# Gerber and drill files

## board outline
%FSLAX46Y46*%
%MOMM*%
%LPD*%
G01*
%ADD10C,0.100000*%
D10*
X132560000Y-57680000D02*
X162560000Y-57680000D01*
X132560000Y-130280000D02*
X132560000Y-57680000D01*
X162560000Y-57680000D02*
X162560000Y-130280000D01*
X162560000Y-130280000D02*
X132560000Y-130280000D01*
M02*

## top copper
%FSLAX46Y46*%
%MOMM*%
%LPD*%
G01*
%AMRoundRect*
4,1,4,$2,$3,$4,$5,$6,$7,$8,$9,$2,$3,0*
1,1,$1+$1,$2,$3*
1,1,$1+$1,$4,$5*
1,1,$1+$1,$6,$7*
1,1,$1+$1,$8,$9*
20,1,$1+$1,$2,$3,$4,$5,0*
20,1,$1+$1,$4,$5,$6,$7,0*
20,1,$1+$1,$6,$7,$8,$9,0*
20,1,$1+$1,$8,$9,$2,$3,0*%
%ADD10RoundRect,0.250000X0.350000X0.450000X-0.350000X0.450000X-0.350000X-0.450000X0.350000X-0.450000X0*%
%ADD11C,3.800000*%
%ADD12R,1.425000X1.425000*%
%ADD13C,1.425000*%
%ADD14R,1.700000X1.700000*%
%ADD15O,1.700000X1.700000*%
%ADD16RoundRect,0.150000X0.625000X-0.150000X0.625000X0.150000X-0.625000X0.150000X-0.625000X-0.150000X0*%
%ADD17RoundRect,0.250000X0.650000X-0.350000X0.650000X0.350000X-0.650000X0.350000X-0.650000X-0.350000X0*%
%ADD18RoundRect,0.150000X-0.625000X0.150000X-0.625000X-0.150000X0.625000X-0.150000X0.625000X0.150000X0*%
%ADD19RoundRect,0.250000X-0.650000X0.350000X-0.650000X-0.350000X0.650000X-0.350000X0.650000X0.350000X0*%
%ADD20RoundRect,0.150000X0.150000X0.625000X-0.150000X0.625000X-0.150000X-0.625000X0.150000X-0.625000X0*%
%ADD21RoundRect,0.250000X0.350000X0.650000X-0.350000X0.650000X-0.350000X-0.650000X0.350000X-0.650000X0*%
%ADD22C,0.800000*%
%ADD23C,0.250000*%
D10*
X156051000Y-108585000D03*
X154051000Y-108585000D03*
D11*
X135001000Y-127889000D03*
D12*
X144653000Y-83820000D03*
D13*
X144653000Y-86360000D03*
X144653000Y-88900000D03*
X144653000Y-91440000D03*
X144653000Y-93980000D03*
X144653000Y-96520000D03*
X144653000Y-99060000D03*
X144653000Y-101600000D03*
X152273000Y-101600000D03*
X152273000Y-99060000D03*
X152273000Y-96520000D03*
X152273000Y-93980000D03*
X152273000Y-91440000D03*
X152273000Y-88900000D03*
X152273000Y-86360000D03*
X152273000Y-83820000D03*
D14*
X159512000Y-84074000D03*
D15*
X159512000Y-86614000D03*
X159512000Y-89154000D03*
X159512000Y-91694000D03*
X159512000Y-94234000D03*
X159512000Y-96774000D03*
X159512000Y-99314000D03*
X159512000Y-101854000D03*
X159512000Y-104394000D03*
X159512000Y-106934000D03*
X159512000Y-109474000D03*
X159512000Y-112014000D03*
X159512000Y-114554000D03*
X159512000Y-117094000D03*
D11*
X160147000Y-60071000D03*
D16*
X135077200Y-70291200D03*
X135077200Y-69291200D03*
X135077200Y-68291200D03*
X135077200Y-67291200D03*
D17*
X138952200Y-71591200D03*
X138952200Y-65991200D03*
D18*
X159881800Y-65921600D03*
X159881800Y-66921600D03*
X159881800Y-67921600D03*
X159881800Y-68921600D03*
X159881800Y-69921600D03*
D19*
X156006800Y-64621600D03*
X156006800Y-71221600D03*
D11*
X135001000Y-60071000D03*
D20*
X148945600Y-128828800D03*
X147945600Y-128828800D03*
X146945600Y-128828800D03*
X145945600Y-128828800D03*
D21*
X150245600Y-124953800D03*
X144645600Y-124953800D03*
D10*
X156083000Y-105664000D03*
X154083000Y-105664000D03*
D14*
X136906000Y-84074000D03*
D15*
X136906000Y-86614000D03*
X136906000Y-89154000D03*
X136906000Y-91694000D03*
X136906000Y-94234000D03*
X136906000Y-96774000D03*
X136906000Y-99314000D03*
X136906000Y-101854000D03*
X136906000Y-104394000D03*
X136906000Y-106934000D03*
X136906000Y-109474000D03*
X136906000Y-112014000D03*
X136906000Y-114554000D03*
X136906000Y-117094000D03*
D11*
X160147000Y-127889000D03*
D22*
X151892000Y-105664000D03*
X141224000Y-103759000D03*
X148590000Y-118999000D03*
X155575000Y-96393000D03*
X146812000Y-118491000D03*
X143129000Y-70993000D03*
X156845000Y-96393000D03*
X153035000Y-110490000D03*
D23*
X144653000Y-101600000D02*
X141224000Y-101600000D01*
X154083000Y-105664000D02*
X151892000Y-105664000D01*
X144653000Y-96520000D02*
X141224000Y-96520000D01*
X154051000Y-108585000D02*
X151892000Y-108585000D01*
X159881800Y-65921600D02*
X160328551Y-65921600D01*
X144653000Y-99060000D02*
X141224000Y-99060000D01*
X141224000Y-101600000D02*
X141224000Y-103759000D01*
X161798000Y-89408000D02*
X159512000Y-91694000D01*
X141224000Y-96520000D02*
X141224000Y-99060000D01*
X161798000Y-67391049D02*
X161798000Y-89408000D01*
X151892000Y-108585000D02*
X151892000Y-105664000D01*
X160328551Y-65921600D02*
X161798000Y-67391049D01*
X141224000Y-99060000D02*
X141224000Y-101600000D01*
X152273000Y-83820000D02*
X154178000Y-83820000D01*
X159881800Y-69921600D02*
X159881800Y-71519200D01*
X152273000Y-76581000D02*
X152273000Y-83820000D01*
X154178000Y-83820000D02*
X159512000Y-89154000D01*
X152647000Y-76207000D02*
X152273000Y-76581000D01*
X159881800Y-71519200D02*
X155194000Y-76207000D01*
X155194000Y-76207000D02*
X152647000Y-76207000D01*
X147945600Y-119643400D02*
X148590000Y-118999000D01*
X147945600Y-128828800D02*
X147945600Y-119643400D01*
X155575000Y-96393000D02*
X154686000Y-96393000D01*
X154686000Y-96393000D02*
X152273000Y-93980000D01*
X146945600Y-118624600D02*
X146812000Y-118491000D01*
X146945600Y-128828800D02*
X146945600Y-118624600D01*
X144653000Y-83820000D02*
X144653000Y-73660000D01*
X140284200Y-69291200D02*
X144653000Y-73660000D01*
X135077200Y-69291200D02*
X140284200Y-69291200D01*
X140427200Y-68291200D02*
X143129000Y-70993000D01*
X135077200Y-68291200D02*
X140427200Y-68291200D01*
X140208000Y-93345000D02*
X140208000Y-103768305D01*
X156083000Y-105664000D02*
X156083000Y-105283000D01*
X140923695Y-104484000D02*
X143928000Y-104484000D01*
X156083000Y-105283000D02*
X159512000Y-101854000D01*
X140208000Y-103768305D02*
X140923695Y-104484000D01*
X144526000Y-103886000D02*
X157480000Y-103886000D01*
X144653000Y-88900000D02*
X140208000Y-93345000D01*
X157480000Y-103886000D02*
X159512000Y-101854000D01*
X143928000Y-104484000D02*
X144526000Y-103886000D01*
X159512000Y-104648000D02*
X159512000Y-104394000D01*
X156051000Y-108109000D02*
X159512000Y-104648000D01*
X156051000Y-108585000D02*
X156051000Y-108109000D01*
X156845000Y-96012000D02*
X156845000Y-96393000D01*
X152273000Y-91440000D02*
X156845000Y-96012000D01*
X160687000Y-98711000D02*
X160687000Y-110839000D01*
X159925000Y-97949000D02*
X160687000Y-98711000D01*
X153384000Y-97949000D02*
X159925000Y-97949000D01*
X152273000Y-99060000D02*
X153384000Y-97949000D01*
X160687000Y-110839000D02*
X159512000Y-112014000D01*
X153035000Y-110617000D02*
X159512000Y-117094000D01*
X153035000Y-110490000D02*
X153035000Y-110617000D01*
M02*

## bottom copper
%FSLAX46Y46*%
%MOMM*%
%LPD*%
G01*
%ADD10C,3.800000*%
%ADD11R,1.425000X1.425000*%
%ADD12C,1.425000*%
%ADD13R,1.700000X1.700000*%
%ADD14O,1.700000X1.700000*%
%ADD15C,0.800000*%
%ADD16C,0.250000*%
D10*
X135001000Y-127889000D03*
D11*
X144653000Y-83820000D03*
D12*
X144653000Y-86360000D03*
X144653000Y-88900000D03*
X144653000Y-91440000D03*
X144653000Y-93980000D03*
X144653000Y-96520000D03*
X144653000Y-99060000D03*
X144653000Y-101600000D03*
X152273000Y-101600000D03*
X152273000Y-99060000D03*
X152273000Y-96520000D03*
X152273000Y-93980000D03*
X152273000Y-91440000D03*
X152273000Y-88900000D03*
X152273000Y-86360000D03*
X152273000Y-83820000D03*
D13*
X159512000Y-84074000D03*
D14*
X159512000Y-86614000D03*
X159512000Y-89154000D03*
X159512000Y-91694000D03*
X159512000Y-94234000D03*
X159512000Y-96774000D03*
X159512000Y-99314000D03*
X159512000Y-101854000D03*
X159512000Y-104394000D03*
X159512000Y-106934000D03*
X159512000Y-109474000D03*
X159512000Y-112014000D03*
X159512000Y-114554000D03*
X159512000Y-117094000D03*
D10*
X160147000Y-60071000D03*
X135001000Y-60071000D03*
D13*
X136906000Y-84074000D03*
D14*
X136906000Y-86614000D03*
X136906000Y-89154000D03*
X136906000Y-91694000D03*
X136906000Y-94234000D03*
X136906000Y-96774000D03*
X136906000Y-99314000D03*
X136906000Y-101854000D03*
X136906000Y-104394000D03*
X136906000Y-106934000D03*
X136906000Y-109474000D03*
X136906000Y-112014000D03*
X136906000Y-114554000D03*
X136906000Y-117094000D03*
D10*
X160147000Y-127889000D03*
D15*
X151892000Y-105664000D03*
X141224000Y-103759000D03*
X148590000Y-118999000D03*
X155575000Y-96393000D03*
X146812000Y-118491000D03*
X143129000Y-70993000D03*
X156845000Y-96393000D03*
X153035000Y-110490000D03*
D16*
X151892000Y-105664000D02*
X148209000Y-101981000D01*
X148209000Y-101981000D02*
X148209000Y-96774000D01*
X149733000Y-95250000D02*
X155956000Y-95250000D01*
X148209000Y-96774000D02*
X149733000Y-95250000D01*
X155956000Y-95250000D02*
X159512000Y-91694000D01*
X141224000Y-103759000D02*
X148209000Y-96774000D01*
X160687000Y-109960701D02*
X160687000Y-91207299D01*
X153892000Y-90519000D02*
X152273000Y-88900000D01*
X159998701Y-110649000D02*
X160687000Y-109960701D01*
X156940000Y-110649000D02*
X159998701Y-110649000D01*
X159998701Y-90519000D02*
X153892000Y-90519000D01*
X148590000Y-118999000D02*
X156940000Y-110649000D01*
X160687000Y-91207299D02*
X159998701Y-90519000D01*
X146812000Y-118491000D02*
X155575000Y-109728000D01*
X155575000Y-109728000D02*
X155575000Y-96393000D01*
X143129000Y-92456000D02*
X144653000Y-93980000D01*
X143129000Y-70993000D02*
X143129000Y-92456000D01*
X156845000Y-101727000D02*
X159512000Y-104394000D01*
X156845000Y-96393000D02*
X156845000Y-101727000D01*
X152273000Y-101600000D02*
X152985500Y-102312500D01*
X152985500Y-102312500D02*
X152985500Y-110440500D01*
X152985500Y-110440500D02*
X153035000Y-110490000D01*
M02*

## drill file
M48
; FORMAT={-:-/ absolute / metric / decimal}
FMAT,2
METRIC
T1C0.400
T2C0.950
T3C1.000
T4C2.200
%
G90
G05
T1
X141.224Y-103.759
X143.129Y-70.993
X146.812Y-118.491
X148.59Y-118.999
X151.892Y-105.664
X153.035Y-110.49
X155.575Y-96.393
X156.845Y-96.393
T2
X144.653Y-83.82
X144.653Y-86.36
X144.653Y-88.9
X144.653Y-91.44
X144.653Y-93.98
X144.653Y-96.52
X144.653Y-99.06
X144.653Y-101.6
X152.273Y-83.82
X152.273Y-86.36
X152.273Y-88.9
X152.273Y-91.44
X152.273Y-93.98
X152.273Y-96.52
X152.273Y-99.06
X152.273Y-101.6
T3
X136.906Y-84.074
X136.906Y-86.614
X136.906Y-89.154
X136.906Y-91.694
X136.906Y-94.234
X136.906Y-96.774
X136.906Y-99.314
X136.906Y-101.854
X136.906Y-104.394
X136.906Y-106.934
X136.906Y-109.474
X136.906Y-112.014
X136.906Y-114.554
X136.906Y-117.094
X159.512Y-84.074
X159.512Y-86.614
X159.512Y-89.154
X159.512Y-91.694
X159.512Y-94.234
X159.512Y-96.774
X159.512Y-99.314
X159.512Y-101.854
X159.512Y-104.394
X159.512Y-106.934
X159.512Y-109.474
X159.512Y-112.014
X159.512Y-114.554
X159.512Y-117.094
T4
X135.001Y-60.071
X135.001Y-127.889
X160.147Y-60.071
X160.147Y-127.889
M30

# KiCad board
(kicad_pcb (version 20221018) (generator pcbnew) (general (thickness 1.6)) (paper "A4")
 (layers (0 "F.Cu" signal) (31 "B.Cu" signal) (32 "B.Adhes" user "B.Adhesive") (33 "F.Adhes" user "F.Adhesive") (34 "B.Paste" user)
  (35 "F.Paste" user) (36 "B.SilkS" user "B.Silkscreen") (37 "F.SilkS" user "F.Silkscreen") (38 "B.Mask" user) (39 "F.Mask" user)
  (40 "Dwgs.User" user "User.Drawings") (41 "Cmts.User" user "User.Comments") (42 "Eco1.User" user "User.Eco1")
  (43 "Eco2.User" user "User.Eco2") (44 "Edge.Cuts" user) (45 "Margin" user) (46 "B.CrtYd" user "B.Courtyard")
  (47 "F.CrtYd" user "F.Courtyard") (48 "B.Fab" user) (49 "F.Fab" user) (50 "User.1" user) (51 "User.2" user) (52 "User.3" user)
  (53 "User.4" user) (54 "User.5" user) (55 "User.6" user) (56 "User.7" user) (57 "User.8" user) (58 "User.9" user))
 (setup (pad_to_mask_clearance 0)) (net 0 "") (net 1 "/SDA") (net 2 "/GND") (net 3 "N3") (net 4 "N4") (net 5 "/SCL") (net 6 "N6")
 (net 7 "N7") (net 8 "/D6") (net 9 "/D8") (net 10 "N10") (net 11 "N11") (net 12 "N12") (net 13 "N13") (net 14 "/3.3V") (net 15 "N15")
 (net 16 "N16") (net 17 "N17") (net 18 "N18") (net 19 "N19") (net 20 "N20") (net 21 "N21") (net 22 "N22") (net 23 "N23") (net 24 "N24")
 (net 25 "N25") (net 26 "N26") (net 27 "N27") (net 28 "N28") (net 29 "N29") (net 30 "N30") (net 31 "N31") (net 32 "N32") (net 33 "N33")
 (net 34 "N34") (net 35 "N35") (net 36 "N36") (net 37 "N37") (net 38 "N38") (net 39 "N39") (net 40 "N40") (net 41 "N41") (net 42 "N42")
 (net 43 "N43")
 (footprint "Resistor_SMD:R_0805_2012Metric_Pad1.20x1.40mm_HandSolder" (layer "F.Cu") (at 155.051 108.585 180)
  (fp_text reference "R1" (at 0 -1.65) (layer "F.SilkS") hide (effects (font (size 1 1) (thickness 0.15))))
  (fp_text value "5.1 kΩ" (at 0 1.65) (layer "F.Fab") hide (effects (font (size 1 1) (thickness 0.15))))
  (pad "1" smd roundrect (at -1 0 180) (size 1.2 1.4) (layers "F.Cu" "F.Paste" "F.Mask") (roundrect_rratio 0.2083333333) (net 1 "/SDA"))
  (pad "2" smd roundrect (at 1 0 180) (size 1.2 1.4) (layers "F.Cu" "F.Paste" "F.Mask") (roundrect_rratio 0.2083333333) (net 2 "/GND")))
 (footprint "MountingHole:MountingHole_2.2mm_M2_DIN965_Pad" (layer "F.Cu") (at 135.001 127.889)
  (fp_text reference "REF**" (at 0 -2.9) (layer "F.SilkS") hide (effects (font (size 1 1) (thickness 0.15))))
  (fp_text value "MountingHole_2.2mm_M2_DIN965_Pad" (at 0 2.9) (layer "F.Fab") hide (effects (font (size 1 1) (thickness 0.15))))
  (pad "1" thru_hole circle (at 0 0) (size 3.8 3.8) (drill 2.2) (layers "*.Cu" "*.Mask")))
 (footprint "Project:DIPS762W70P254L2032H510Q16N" (layer "F.Cu") (at 144.653 83.82)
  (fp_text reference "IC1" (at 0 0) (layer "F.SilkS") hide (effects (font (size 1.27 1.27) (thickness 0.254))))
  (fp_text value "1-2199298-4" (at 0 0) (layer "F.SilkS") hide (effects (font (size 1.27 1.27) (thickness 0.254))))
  (pad "1" thru_hole rect (at 0 0) (size 1.425 1.425) (drill 0.95) (layers "*.Cu" "*.Mask") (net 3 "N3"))
  (pad "2" thru_hole circle (at 0 2.54) (size 1.425 1.425) (drill 0.95) (layers "*.Cu" "*.Mask") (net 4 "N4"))
  (pad "3" thru_hole circle (at 0 5.08) (size 1.425 1.425) (drill 0.95) (layers "*.Cu" "*.Mask") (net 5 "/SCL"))
  (pad "4" thru_hole circle (at 0 7.62) (size 1.425 1.425) (drill 0.95) (layers "*.Cu" "*.Mask") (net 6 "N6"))
  (pad "5" thru_hole circle (at 0 10.16) (size 1.425 1.425) (drill 0.95) (layers "*.Cu" "*.Mask") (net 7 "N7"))
  (pad "6" thru_hole circle (at 0 12.7) (size 1.425 1.425) (drill 0.95) (layers "*.Cu" "*.Mask") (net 2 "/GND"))
  (pad "7" thru_hole circle (at 0 15.24) (size 1.425 1.425) (drill 0.95) (layers "*.Cu" "*.Mask") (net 2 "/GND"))
  (pad "8" thru_hole circle (at 0 17.78) (size 1.425 1.425) (drill 0.95) (layers "*.Cu" "*.Mask") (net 2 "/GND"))
  (pad "9" thru_hole circle (at 7.62 17.78) (size 1.425 1.425) (drill 0.95) (layers "*.Cu" "*.Mask") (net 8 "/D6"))
  (pad "10" thru_hole circle (at 7.62 15.24) (size 1.425 1.425) (drill 0.95) (layers "*.Cu" "*.Mask") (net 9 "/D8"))
  (pad "11" thru_hole circle (at 7.62 12.7) (size 1.425 1.425) (drill 0.95) (layers "*.Cu" "*.Mask") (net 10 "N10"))
  (pad "12" thru_hole circle (at 7.62 10.16) (size 1.425 1.425) (drill 0.95) (layers "*.Cu" "*.Mask") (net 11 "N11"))
  (pad "13" thru_hole circle (at 7.62 7.62) (size 1.425 1.425) (drill 0.95) (layers "*.Cu" "*.Mask") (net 1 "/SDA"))
  (pad "14" thru_hole circle (at 7.62 5.08) (size 1.425 1.425) (drill 0.95) (layers "*.Cu" "*.Mask") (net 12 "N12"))
  (pad "15" thru_hole circle (at 7.62 2.54) (size 1.425 1.425) (drill 0.95) (layers "*.Cu" "*.Mask") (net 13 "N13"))
  (pad "16" thru_hole circle (at 7.62 0) (size 1.425 1.425) (drill 0.95) (layers "*.Cu" "*.Mask") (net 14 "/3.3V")))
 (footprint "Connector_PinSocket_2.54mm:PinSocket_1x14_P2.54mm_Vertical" (layer "F.Cu") (at 159.512 84.074)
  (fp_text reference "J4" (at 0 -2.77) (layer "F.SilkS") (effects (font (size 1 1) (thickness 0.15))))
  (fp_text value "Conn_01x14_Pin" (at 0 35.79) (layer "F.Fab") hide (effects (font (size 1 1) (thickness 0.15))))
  (pad "1" thru_hole rect (at 0 0) (size 1.7 1.7) (drill 1) (layers "*.Cu" "*.Mask") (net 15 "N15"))
  (pad "2" thru_hole oval (at 0 2.54) (size 1.7 1.7) (drill 1) (layers "*.Cu" "*.Mask") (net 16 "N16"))
  (pad "3" thru_hole oval (at 0 5.08) (size 1.7 1.7) (drill 1) (layers "*.Cu" "*.Mask") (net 14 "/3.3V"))
  (pad "4" thru_hole oval (at 0 7.62) (size 1.7 1.7) (drill 1) (layers "*.Cu" "*.Mask") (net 2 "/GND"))
  (pad "5" thru_hole oval (at 0 10.16) (size 1.7 1.7) (drill 1) (layers "*.Cu" "*.Mask") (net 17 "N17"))
  (pad "6" thru_hole oval (at 0 12.7) (size 1.7 1.7) (drill 1) (layers "*.Cu" "*.Mask") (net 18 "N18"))
  (pad "7" thru_hole oval (at 0 15.24) (size 1.7 1.7) (drill 1) (layers "*.Cu" "*.Mask") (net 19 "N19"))
  (pad "8" thru_hole oval (at 0 17.78) (size 1.7 1.7) (drill 1) (layers "*.Cu" "*.Mask") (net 5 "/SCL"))
  (pad "9" thru_hole oval (at 0 20.32) (size 1.7 1.7) (drill 1) (layers "*.Cu" "*.Mask") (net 1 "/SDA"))
  (pad "10" thru_hole oval (at 0 22.86) (size 1.7 1.7) (drill 1) (layers "*.Cu" "*.Mask") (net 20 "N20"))
  (pad "11" thru_hole oval (at 0 25.4) (size 1.7 1.7) (drill 1) (layers "*.Cu" "*.Mask") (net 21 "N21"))
  (pad "12" thru_hole oval (at 0 27.94) (size 1.7 1.7) (drill 1) (layers "*.Cu" "*.Mask") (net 9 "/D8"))
  (pad "13" thru_hole oval (at 0 30.48) (size 1.7 1.7) (drill 1) (layers "*.Cu" "*.Mask") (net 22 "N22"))
  (pad "14" thru_hole oval (at 0 33.02) (size 1.7 1.7) (drill 1) (layers "*.Cu" "*.Mask") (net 8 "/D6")))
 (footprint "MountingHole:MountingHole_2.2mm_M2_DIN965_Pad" (layer "F.Cu") (at 160.147 60.071)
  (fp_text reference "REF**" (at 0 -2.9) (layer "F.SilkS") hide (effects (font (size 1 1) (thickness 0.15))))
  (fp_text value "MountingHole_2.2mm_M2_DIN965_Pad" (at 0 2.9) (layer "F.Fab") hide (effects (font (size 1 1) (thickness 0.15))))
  (pad "1" thru_hole circle (at 0 0) (size 3.8 3.8) (drill 2.2) (layers "*.Cu" "*.Mask")))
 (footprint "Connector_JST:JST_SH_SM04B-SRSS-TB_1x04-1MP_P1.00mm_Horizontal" (layer "F.Cu") (at 137.0772 68.7912 90)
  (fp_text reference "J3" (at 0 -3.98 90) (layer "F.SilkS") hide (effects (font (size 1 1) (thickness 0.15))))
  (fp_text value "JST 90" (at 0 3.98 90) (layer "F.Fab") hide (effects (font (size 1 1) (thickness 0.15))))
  (pad "1" smd roundrect (at -1.5 -2 90) (size 0.6 1.55) (layers "F.Cu" "F.Paste" "F.Mask") (roundrect_rratio 0.25) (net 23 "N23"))
  (pad "2" smd roundrect (at -0.5 -2 90) (size 0.6 1.55) (layers "F.Cu" "F.Paste" "F.Mask") (roundrect_rratio 0.25) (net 3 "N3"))
  (pad "3" smd roundrect (at 0.5 -2 90) (size 0.6 1.55) (layers "F.Cu" "F.Paste" "F.Mask") (roundrect_rratio 0.25) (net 7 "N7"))
  (pad "4" smd roundrect (at 1.5 -2 90) (size 0.6 1.55) (layers "F.Cu" "F.Paste" "F.Mask") (roundrect_rratio 0.25) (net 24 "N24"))
  (pad "MP" smd roundrect (at -2.8 1.875 90) (size 1.2 1.8) (layers "F.Cu" "F.Paste" "F.Mask") (roundrect_rratio 0.208333))
  (pad "MP" smd roundrect (at 2.8 1.875 90) (size 1.2 1.8) (layers "F.Cu" "F.Paste" "F.Mask") (roundrect_rratio 0.208333)))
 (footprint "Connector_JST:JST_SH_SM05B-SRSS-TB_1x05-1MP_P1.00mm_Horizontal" (layer "F.Cu") (at 157.8818 67.9216 -90)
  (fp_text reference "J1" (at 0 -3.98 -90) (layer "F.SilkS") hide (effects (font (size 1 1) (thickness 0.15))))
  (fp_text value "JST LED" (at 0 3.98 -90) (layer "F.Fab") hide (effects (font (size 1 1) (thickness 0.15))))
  (pad "1" smd roundrect (at -2 -2 270) (size 0.6 1.55) (layers "F.Cu" "F.Paste" "F.Mask") (roundrect_rratio 0.25) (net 2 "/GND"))
  (pad "2" smd roundrect (at -1 -2 270) (size 0.6 1.55) (layers "F.Cu" "F.Paste" "F.Mask") (roundrect_rratio 0.25) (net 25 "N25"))
  (pad "3" smd roundrect (at 0 -2 270) (size 0.6 1.55) (layers "F.Cu" "F.Paste" "F.Mask") (roundrect_rratio 0.25) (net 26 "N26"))
  (pad "4" smd roundrect (at 1 -2 270) (size 0.6 1.55) (layers "F.Cu" "F.Paste" "F.Mask") (roundrect_rratio 0.25) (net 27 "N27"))
  (pad "5" smd roundrect (at 2 -2 270) (size 0.6 1.55) (layers "F.Cu" "F.Paste" "F.Mask") (roundrect_rratio 0.25) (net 14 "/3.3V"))
  (pad "MP" smd roundrect (at -3.3 1.875 270) (size 1.2 1.8) (layers "F.Cu" "F.Paste" "F.Mask") (roundrect_rratio 0.208333))
  (pad "MP" smd roundrect (at 3.3 1.875 270) (size 1.2 1.8) (layers "F.Cu" "F.Paste" "F.Mask") (roundrect_rratio 0.208333)))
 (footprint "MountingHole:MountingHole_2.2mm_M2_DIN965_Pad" (layer "F.Cu") (at 135.001 60.071)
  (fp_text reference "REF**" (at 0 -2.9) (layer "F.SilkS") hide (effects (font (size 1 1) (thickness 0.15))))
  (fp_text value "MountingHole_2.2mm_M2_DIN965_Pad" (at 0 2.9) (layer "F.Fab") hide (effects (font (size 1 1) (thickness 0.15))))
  (pad "1" thru_hole circle (at 0 0) (size 3.8 3.8) (drill 2.2) (layers "*.Cu" "*.Mask")))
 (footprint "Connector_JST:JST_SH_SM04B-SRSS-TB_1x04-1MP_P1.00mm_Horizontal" (layer "F.Cu") (at 147.4456 126.8288 180)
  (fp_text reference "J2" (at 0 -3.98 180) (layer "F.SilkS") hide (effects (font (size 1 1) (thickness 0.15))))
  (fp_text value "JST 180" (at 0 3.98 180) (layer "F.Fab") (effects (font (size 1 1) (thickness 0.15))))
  (pad "1" smd roundrect (at -1.5 -2 180) (size 0.6 1.55) (layers "F.Cu" "F.Paste" "F.Mask") (roundrect_rratio 0.25) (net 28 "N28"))
  (pad "2" smd roundrect (at -0.5 -2 180) (size 0.6 1.55) (layers "F.Cu" "F.Paste" "F.Mask") (roundrect_rratio 0.25) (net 12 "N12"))
  (pad "3" smd roundrect (at 0.5 -2 180) (size 0.6 1.55) (layers "F.Cu" "F.Paste" "F.Mask") (roundrect_rratio 0.25) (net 11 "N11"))
  (pad "4" smd roundrect (at 1.5 -2 180) (size 0.6 1.55) (layers "F.Cu" "F.Paste" "F.Mask") (roundrect_rratio 0.25) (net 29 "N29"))
  (pad "MP" smd roundrect (at -2.8 1.875 180) (size 1.2 1.8) (layers "F.Cu" "F.Paste" "F.Mask") (roundrect_rratio 0.208333))
  (pad "MP" smd roundrect (at 2.8 1.875 180) (size 1.2 1.8) (layers "F.Cu" "F.Paste" "F.Mask") (roundrect_rratio 0.208333)))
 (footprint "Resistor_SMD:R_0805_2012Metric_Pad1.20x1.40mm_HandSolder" (layer "F.Cu") (at 155.083 105.664 180)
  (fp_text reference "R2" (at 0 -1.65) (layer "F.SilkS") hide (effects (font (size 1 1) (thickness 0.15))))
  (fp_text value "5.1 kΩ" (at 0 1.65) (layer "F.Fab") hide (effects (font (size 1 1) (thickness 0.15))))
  (pad "1" smd roundrect (at -1 0 180) (size 1.2 1.4) (layers "F.Cu" "F.Paste" "F.Mask") (roundrect_rratio 0.2083333333) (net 5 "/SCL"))
  (pad "2" smd roundrect (at 1 0 180) (size 1.2 1.4) (layers "F.Cu" "F.Paste" "F.Mask") (roundrect_rratio 0.2083333333) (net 2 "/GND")))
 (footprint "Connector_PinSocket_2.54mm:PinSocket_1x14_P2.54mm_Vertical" (layer "F.Cu") (at 136.906 84.074)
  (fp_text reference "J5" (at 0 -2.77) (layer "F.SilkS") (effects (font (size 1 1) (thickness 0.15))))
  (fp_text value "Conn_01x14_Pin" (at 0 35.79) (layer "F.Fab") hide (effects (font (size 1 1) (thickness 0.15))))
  (pad "1" thru_hole rect (at 0 0) (size 1.7 1.7) (drill 1) (layers "*.Cu" "*.Mask") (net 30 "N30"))
  (pad "2" thru_hole oval (at 0 2.54) (size 1.7 1.7) (drill 1) (layers "*.Cu" "*.Mask") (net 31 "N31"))
  (pad "3" thru_hole oval (at 0 5.08) (size 1.7 1.7) (drill 1) (layers "*.Cu" "*.Mask") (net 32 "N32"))
  (pad "4" thru_hole oval (at 0 7.62) (size 1.7 1.7) (drill 1) (layers "*.Cu" "*.Mask") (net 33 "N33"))
  (pad "5" thru_hole oval (at 0 10.16) (size 1.7 1.7) (drill 1) (layers "*.Cu" "*.Mask") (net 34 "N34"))
  (pad "6" thru_hole oval (at 0 12.7) (size 1.7 1.7) (drill 1) (layers "*.Cu" "*.Mask") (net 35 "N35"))
  (pad "7" thru_hole oval (at 0 15.24) (size 1.7 1.7) (drill 1) (layers "*.Cu" "*.Mask") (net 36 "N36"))
  (pad "8" thru_hole oval (at 0 17.78) (size 1.7 1.7) (drill 1) (layers "*.Cu" "*.Mask") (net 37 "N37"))
  (pad "9" thru_hole oval (at 0 20.32) (size 1.7 1.7) (drill 1) (layers "*.Cu" "*.Mask") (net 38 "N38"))
  (pad "10" thru_hole oval (at 0 22.86) (size 1.7 1.7) (drill 1) (layers "*.Cu" "*.Mask") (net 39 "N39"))
  (pad "11" thru_hole oval (at 0 25.4) (size 1.7 1.7) (drill 1) (layers "*.Cu" "*.Mask") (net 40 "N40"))
  (pad "12" thru_hole oval (at 0 27.94) (size 1.7 1.7) (drill 1) (layers "*.Cu" "*.Mask") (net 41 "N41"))
  (pad "13" thru_hole oval (at 0 30.48) (size 1.7 1.7) (drill 1) (layers "*.Cu" "*.Mask") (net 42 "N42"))
  (pad "14" thru_hole oval (at 0 33.02) (size 1.7 1.7) (drill 1) (layers "*.Cu" "*.Mask") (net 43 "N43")))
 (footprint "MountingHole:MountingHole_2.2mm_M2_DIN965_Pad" (layer "F.Cu") (at 160.147 127.889)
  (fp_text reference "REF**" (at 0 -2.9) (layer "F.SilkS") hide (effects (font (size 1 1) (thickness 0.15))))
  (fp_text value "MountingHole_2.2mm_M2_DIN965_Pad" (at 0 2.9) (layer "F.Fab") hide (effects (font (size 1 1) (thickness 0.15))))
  (pad "1" thru_hole circle (at 0 0) (size 3.8 3.8) (drill 2.2) (layers "*.Cu" "*.Mask")))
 (gr_line (start 132.56 57.68) (end 162.56 57.68) (stroke (width 0.1) (type default)) (layer "Edge.Cuts"))
 (gr_line (start 132.56 130.28) (end 132.56 57.68) (stroke (width 0.1) (type default)) (layer "Edge.Cuts"))
 (gr_line (start 162.56 57.68) (end 162.56 130.28) (stroke (width 0.1) (type default)) (layer "Edge.Cuts"))
 (gr_line (start 162.56 130.28) (end 132.56 130.28) (stroke (width 0.1) (type default)) (layer "Edge.Cuts"))
 (segment (start 144.653 101.6) (end 141.224 101.6) (width 0.25) (layer "F.Cu") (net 2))
 (segment (start 154.083 105.664) (end 151.892 105.664) (width 0.25) (layer "F.Cu") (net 2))
 (segment (start 144.653 96.52) (end 141.224 96.52) (width 0.25) (layer "F.Cu") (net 2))
 (segment (start 154.051 108.585) (end 151.892 108.585) (width 0.25) (layer "F.Cu") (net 2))
 (segment (start 159.8818 65.9216) (end 160.328551 65.9216) (width 0.25) (layer "F.Cu") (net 2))
 (segment (start 144.653 99.06) (end 141.224 99.06) (width 0.25) (layer "F.Cu") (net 2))
 (segment (start 141.224 101.6) (end 141.224 103.759) (width 0.25) (layer "F.Cu") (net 2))
 (segment (start 161.798 89.408) (end 159.512 91.694) (width 0.25) (layer "F.Cu") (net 2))
 (segment (start 141.224 96.52) (end 141.224 99.06) (width 0.25) (layer "F.Cu") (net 2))
 (segment (start 161.798 67.391049) (end 161.798 89.408) (width 0.25) (layer "F.Cu") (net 2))
 (segment (start 151.892 108.585) (end 151.892 105.664) (width 0.25) (layer "F.Cu") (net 2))
 (segment (start 160.328551 65.9216) (end 161.798 67.391049) (width 0.25) (layer "F.Cu") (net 2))
 (segment (start 141.224 99.06) (end 141.224 101.6) (width 0.25) (layer "F.Cu") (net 2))
 (via (at 151.892 105.664) (size 0.8) (drill 0.4) (layers "F.Cu" "B.Cu") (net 2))
 (via (at 141.224 103.759) (size 0.8) (drill 0.4) (layers "F.Cu" "B.Cu") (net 2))
 (segment (start 151.892 105.664) (end 148.209 101.981) (width 0.25) (layer "B.Cu") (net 2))
 (segment (start 148.209 101.981) (end 148.209 96.774) (width 0.25) (layer "B.Cu") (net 2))
 (segment (start 149.733 95.25) (end 155.956 95.25) (width 0.25) (layer "B.Cu") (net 2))
 (segment (start 148.209 96.774) (end 149.733 95.25) (width 0.25) (layer "B.Cu") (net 2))
 (segment (start 155.956 95.25) (end 159.512 91.694) (width 0.25) (layer "B.Cu") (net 2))
 (segment (start 141.224 103.759) (end 148.209 96.774) (width 0.25) (layer "B.Cu") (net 2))
 (segment (start 152.273 83.82) (end 154.178 83.82) (width 0.25) (layer "F.Cu") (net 14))
 (segment (start 159.8818 69.9216) (end 159.8818 71.5192) (width 0.25) (layer "F.Cu") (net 14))
 (segment (start 152.273 76.581) (end 152.273 83.82) (width 0.25) (layer "F.Cu") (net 14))
 (segment (start 154.178 83.82) (end 159.512 89.154) (width 0.25) (layer "F.Cu") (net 14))
 (segment (start 152.647 76.207) (end 152.273 76.581) (width 0.25) (layer "F.Cu") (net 14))
 (segment (start 159.8818 71.5192) (end 155.194 76.207) (width 0.25) (layer "F.Cu") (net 14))
 (segment (start 155.194 76.207) (end 152.647 76.207) (width 0.25) (layer "F.Cu") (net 14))
 (segment (start 147.9456 119.6434) (end 148.59 118.999) (width 0.25) (layer "F.Cu") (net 12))
 (segment (start 147.9456 128.8288) (end 147.9456 119.6434) (width 0.25) (layer "F.Cu") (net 12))
 (via (at 148.59 118.999) (size 0.8) (drill 0.4) (layers "F.Cu" "B.Cu") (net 12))
 (segment (start 160.687 109.960701) (end 160.687 91.207299) (width 0.25) (layer "B.Cu") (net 12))
 (segment (start 153.892 90.519) (end 152.273 88.9) (width 0.25) (layer "B.Cu") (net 12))
 (segment (start 159.998701 110.649) (end 160.687 109.960701) (width 0.25) (layer "B.Cu") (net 12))
 (segment (start 156.94 110.649) (end 159.998701 110.649) (width 0.25) (layer "B.Cu") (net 12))
 (segment (start 159.998701 90.519) (end 153.892 90.519) (width 0.25) (layer "B.Cu") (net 12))
 (segment (start 148.59 118.999) (end 156.94 110.649) (width 0.25) (layer "B.Cu") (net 12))
 (segment (start 160.687 91.207299) (end 159.998701 90.519) (width 0.25) (layer "B.Cu") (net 12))
 (segment (start 155.575 96.393) (end 154.686 96.393) (width 0.25) (layer "F.Cu") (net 11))
 (segment (start 154.686 96.393) (end 152.273 93.98) (width 0.25) (layer "F.Cu") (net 11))
 (segment (start 146.9456 118.6246) (end 146.812 118.491) (width 0.25) (layer "F.Cu") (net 11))
 (segment (start 146.9456 128.8288) (end 146.9456 118.6246) (width 0.25) (layer "F.Cu") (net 11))
 (via (at 155.575 96.393) (size 0.8) (drill 0.4) (layers "F.Cu" "B.Cu") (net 11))
 (via (at 146.812 118.491) (size 0.8) (drill 0.4) (layers "F.Cu" "B.Cu") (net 11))
 (segment (start 146.812 118.491) (end 155.575 109.728) (width 0.25) (layer "B.Cu") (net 11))
 (segment (start 155.575 109.728) (end 155.575 96.393) (width 0.25) (layer "B.Cu") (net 11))
 (segment (start 144.653 83.82) (end 144.653 73.66) (width 0.25) (layer "F.Cu") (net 3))
 (segment (start 140.2842 69.2912) (end 144.653 73.66) (width 0.25) (layer "F.Cu") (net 3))
 (segment (start 135.0772 69.2912) (end 140.2842 69.2912) (width 0.25) (layer "F.Cu") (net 3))
 (segment (start 140.4272 68.2912) (end 143.129 70.993) (width 0.25) (layer "F.Cu") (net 7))
 (segment (start 135.0772 68.2912) (end 140.4272 68.2912) (width 0.25) (layer "F.Cu") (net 7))
 (via (at 143.129 70.993) (size 0.8) (drill 0.4) (layers "F.Cu" "B.Cu") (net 7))
 (segment (start 143.129 92.456) (end 144.653 93.98) (width 0.25) (layer "B.Cu") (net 7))
 (segment (start 143.129 70.993) (end 143.129 92.456) (width 0.25) (layer "B.Cu") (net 7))
 (segment (start 140.208 93.345) (end 140.208 103.768305) (width 0.25) (layer "F.Cu") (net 5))
 (segment (start 156.083 105.664) (end 156.083 105.283) (width 0.25) (layer "F.Cu") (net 5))
 (segment (start 140.923695 104.484) (end 143.928 104.484) (width 0.25) (layer "F.Cu") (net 5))
 (segment (start 156.083 105.283) (end 159.512 101.854) (width 0.25) (layer "F.Cu") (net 5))
 (segment (start 140.208 103.768305) (end 140.923695 104.484) (width 0.25) (layer "F.Cu") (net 5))
 (segment (start 144.526 103.886) (end 157.48 103.886) (width 0.25) (layer "F.Cu") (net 5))
 (segment (start 144.653 88.9) (end 140.208 93.345) (width 0.25) (layer "F.Cu") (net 5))
 (segment (start 157.48 103.886) (end 159.512 101.854) (width 0.25) (layer "F.Cu") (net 5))
 (segment (start 143.928 104.484) (end 144.526 103.886) (width 0.25) (layer "F.Cu") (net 5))
 (segment (start 159.512 104.648) (end 159.512 104.394) (width 0.25) (layer "F.Cu") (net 1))
 (segment (start 156.051 108.109) (end 159.512 104.648) (width 0.25) (layer "F.Cu") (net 1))
 (segment (start 156.051 108.585) (end 156.051 108.109) (width 0.25) (layer "F.Cu") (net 1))
 (segment (start 156.845 96.012) (end 156.845 96.393) (width 0.25) (layer "F.Cu") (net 1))
 (segment (start 152.273 91.44) (end 156.845 96.012) (width 0.25) (layer "F.Cu") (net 1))
 (via (at 156.845 96.393) (size 0.8) (drill 0.4) (layers "F.Cu" "B.Cu") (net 1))
 (segment (start 156.845 101.727) (end 159.512 104.394) (width 0.25) (layer "B.Cu") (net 1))
 (segment (start 156.845 96.393) (end 156.845 101.727) (width 0.25) (layer "B.Cu") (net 1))
 (segment (start 160.687 98.711) (end 160.687 110.839) (width 0.25) (layer "F.Cu") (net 9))
 (segment (start 159.925 97.949) (end 160.687 98.711) (width 0.25) (layer "F.Cu") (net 9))
 (segment (start 153.384 97.949) (end 159.925 97.949) (width 0.25) (layer "F.Cu") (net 9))
 (segment (start 152.273 99.06) (end 153.384 97.949) (width 0.25) (layer "F.Cu") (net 9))
 (segment (start 160.687 110.839) (end 159.512 112.014) (width 0.25) (layer "F.Cu") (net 9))
 (segment (start 153.035 110.617) (end 159.512 117.094) (width 0.25) (layer "F.Cu") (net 8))
 (segment (start 153.035 110.49) (end 153.035 110.617) (width 0.25) (layer "F.Cu") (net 8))
 (via (at 153.035 110.49) (size 0.8) (drill 0.4) (layers "F.Cu" "B.Cu") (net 8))
 (segment (start 152.273 101.6) (end 152.9855 102.3125) (width 0.25) (layer "B.Cu") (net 8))
 (segment (start 152.9855 102.3125) (end 152.9855 110.4405) (width 0.25) (layer "B.Cu") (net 8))
 (segment (start 152.9855 110.4405) (end 153.035 110.49) (width 0.25) (layer "B.Cu") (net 8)))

